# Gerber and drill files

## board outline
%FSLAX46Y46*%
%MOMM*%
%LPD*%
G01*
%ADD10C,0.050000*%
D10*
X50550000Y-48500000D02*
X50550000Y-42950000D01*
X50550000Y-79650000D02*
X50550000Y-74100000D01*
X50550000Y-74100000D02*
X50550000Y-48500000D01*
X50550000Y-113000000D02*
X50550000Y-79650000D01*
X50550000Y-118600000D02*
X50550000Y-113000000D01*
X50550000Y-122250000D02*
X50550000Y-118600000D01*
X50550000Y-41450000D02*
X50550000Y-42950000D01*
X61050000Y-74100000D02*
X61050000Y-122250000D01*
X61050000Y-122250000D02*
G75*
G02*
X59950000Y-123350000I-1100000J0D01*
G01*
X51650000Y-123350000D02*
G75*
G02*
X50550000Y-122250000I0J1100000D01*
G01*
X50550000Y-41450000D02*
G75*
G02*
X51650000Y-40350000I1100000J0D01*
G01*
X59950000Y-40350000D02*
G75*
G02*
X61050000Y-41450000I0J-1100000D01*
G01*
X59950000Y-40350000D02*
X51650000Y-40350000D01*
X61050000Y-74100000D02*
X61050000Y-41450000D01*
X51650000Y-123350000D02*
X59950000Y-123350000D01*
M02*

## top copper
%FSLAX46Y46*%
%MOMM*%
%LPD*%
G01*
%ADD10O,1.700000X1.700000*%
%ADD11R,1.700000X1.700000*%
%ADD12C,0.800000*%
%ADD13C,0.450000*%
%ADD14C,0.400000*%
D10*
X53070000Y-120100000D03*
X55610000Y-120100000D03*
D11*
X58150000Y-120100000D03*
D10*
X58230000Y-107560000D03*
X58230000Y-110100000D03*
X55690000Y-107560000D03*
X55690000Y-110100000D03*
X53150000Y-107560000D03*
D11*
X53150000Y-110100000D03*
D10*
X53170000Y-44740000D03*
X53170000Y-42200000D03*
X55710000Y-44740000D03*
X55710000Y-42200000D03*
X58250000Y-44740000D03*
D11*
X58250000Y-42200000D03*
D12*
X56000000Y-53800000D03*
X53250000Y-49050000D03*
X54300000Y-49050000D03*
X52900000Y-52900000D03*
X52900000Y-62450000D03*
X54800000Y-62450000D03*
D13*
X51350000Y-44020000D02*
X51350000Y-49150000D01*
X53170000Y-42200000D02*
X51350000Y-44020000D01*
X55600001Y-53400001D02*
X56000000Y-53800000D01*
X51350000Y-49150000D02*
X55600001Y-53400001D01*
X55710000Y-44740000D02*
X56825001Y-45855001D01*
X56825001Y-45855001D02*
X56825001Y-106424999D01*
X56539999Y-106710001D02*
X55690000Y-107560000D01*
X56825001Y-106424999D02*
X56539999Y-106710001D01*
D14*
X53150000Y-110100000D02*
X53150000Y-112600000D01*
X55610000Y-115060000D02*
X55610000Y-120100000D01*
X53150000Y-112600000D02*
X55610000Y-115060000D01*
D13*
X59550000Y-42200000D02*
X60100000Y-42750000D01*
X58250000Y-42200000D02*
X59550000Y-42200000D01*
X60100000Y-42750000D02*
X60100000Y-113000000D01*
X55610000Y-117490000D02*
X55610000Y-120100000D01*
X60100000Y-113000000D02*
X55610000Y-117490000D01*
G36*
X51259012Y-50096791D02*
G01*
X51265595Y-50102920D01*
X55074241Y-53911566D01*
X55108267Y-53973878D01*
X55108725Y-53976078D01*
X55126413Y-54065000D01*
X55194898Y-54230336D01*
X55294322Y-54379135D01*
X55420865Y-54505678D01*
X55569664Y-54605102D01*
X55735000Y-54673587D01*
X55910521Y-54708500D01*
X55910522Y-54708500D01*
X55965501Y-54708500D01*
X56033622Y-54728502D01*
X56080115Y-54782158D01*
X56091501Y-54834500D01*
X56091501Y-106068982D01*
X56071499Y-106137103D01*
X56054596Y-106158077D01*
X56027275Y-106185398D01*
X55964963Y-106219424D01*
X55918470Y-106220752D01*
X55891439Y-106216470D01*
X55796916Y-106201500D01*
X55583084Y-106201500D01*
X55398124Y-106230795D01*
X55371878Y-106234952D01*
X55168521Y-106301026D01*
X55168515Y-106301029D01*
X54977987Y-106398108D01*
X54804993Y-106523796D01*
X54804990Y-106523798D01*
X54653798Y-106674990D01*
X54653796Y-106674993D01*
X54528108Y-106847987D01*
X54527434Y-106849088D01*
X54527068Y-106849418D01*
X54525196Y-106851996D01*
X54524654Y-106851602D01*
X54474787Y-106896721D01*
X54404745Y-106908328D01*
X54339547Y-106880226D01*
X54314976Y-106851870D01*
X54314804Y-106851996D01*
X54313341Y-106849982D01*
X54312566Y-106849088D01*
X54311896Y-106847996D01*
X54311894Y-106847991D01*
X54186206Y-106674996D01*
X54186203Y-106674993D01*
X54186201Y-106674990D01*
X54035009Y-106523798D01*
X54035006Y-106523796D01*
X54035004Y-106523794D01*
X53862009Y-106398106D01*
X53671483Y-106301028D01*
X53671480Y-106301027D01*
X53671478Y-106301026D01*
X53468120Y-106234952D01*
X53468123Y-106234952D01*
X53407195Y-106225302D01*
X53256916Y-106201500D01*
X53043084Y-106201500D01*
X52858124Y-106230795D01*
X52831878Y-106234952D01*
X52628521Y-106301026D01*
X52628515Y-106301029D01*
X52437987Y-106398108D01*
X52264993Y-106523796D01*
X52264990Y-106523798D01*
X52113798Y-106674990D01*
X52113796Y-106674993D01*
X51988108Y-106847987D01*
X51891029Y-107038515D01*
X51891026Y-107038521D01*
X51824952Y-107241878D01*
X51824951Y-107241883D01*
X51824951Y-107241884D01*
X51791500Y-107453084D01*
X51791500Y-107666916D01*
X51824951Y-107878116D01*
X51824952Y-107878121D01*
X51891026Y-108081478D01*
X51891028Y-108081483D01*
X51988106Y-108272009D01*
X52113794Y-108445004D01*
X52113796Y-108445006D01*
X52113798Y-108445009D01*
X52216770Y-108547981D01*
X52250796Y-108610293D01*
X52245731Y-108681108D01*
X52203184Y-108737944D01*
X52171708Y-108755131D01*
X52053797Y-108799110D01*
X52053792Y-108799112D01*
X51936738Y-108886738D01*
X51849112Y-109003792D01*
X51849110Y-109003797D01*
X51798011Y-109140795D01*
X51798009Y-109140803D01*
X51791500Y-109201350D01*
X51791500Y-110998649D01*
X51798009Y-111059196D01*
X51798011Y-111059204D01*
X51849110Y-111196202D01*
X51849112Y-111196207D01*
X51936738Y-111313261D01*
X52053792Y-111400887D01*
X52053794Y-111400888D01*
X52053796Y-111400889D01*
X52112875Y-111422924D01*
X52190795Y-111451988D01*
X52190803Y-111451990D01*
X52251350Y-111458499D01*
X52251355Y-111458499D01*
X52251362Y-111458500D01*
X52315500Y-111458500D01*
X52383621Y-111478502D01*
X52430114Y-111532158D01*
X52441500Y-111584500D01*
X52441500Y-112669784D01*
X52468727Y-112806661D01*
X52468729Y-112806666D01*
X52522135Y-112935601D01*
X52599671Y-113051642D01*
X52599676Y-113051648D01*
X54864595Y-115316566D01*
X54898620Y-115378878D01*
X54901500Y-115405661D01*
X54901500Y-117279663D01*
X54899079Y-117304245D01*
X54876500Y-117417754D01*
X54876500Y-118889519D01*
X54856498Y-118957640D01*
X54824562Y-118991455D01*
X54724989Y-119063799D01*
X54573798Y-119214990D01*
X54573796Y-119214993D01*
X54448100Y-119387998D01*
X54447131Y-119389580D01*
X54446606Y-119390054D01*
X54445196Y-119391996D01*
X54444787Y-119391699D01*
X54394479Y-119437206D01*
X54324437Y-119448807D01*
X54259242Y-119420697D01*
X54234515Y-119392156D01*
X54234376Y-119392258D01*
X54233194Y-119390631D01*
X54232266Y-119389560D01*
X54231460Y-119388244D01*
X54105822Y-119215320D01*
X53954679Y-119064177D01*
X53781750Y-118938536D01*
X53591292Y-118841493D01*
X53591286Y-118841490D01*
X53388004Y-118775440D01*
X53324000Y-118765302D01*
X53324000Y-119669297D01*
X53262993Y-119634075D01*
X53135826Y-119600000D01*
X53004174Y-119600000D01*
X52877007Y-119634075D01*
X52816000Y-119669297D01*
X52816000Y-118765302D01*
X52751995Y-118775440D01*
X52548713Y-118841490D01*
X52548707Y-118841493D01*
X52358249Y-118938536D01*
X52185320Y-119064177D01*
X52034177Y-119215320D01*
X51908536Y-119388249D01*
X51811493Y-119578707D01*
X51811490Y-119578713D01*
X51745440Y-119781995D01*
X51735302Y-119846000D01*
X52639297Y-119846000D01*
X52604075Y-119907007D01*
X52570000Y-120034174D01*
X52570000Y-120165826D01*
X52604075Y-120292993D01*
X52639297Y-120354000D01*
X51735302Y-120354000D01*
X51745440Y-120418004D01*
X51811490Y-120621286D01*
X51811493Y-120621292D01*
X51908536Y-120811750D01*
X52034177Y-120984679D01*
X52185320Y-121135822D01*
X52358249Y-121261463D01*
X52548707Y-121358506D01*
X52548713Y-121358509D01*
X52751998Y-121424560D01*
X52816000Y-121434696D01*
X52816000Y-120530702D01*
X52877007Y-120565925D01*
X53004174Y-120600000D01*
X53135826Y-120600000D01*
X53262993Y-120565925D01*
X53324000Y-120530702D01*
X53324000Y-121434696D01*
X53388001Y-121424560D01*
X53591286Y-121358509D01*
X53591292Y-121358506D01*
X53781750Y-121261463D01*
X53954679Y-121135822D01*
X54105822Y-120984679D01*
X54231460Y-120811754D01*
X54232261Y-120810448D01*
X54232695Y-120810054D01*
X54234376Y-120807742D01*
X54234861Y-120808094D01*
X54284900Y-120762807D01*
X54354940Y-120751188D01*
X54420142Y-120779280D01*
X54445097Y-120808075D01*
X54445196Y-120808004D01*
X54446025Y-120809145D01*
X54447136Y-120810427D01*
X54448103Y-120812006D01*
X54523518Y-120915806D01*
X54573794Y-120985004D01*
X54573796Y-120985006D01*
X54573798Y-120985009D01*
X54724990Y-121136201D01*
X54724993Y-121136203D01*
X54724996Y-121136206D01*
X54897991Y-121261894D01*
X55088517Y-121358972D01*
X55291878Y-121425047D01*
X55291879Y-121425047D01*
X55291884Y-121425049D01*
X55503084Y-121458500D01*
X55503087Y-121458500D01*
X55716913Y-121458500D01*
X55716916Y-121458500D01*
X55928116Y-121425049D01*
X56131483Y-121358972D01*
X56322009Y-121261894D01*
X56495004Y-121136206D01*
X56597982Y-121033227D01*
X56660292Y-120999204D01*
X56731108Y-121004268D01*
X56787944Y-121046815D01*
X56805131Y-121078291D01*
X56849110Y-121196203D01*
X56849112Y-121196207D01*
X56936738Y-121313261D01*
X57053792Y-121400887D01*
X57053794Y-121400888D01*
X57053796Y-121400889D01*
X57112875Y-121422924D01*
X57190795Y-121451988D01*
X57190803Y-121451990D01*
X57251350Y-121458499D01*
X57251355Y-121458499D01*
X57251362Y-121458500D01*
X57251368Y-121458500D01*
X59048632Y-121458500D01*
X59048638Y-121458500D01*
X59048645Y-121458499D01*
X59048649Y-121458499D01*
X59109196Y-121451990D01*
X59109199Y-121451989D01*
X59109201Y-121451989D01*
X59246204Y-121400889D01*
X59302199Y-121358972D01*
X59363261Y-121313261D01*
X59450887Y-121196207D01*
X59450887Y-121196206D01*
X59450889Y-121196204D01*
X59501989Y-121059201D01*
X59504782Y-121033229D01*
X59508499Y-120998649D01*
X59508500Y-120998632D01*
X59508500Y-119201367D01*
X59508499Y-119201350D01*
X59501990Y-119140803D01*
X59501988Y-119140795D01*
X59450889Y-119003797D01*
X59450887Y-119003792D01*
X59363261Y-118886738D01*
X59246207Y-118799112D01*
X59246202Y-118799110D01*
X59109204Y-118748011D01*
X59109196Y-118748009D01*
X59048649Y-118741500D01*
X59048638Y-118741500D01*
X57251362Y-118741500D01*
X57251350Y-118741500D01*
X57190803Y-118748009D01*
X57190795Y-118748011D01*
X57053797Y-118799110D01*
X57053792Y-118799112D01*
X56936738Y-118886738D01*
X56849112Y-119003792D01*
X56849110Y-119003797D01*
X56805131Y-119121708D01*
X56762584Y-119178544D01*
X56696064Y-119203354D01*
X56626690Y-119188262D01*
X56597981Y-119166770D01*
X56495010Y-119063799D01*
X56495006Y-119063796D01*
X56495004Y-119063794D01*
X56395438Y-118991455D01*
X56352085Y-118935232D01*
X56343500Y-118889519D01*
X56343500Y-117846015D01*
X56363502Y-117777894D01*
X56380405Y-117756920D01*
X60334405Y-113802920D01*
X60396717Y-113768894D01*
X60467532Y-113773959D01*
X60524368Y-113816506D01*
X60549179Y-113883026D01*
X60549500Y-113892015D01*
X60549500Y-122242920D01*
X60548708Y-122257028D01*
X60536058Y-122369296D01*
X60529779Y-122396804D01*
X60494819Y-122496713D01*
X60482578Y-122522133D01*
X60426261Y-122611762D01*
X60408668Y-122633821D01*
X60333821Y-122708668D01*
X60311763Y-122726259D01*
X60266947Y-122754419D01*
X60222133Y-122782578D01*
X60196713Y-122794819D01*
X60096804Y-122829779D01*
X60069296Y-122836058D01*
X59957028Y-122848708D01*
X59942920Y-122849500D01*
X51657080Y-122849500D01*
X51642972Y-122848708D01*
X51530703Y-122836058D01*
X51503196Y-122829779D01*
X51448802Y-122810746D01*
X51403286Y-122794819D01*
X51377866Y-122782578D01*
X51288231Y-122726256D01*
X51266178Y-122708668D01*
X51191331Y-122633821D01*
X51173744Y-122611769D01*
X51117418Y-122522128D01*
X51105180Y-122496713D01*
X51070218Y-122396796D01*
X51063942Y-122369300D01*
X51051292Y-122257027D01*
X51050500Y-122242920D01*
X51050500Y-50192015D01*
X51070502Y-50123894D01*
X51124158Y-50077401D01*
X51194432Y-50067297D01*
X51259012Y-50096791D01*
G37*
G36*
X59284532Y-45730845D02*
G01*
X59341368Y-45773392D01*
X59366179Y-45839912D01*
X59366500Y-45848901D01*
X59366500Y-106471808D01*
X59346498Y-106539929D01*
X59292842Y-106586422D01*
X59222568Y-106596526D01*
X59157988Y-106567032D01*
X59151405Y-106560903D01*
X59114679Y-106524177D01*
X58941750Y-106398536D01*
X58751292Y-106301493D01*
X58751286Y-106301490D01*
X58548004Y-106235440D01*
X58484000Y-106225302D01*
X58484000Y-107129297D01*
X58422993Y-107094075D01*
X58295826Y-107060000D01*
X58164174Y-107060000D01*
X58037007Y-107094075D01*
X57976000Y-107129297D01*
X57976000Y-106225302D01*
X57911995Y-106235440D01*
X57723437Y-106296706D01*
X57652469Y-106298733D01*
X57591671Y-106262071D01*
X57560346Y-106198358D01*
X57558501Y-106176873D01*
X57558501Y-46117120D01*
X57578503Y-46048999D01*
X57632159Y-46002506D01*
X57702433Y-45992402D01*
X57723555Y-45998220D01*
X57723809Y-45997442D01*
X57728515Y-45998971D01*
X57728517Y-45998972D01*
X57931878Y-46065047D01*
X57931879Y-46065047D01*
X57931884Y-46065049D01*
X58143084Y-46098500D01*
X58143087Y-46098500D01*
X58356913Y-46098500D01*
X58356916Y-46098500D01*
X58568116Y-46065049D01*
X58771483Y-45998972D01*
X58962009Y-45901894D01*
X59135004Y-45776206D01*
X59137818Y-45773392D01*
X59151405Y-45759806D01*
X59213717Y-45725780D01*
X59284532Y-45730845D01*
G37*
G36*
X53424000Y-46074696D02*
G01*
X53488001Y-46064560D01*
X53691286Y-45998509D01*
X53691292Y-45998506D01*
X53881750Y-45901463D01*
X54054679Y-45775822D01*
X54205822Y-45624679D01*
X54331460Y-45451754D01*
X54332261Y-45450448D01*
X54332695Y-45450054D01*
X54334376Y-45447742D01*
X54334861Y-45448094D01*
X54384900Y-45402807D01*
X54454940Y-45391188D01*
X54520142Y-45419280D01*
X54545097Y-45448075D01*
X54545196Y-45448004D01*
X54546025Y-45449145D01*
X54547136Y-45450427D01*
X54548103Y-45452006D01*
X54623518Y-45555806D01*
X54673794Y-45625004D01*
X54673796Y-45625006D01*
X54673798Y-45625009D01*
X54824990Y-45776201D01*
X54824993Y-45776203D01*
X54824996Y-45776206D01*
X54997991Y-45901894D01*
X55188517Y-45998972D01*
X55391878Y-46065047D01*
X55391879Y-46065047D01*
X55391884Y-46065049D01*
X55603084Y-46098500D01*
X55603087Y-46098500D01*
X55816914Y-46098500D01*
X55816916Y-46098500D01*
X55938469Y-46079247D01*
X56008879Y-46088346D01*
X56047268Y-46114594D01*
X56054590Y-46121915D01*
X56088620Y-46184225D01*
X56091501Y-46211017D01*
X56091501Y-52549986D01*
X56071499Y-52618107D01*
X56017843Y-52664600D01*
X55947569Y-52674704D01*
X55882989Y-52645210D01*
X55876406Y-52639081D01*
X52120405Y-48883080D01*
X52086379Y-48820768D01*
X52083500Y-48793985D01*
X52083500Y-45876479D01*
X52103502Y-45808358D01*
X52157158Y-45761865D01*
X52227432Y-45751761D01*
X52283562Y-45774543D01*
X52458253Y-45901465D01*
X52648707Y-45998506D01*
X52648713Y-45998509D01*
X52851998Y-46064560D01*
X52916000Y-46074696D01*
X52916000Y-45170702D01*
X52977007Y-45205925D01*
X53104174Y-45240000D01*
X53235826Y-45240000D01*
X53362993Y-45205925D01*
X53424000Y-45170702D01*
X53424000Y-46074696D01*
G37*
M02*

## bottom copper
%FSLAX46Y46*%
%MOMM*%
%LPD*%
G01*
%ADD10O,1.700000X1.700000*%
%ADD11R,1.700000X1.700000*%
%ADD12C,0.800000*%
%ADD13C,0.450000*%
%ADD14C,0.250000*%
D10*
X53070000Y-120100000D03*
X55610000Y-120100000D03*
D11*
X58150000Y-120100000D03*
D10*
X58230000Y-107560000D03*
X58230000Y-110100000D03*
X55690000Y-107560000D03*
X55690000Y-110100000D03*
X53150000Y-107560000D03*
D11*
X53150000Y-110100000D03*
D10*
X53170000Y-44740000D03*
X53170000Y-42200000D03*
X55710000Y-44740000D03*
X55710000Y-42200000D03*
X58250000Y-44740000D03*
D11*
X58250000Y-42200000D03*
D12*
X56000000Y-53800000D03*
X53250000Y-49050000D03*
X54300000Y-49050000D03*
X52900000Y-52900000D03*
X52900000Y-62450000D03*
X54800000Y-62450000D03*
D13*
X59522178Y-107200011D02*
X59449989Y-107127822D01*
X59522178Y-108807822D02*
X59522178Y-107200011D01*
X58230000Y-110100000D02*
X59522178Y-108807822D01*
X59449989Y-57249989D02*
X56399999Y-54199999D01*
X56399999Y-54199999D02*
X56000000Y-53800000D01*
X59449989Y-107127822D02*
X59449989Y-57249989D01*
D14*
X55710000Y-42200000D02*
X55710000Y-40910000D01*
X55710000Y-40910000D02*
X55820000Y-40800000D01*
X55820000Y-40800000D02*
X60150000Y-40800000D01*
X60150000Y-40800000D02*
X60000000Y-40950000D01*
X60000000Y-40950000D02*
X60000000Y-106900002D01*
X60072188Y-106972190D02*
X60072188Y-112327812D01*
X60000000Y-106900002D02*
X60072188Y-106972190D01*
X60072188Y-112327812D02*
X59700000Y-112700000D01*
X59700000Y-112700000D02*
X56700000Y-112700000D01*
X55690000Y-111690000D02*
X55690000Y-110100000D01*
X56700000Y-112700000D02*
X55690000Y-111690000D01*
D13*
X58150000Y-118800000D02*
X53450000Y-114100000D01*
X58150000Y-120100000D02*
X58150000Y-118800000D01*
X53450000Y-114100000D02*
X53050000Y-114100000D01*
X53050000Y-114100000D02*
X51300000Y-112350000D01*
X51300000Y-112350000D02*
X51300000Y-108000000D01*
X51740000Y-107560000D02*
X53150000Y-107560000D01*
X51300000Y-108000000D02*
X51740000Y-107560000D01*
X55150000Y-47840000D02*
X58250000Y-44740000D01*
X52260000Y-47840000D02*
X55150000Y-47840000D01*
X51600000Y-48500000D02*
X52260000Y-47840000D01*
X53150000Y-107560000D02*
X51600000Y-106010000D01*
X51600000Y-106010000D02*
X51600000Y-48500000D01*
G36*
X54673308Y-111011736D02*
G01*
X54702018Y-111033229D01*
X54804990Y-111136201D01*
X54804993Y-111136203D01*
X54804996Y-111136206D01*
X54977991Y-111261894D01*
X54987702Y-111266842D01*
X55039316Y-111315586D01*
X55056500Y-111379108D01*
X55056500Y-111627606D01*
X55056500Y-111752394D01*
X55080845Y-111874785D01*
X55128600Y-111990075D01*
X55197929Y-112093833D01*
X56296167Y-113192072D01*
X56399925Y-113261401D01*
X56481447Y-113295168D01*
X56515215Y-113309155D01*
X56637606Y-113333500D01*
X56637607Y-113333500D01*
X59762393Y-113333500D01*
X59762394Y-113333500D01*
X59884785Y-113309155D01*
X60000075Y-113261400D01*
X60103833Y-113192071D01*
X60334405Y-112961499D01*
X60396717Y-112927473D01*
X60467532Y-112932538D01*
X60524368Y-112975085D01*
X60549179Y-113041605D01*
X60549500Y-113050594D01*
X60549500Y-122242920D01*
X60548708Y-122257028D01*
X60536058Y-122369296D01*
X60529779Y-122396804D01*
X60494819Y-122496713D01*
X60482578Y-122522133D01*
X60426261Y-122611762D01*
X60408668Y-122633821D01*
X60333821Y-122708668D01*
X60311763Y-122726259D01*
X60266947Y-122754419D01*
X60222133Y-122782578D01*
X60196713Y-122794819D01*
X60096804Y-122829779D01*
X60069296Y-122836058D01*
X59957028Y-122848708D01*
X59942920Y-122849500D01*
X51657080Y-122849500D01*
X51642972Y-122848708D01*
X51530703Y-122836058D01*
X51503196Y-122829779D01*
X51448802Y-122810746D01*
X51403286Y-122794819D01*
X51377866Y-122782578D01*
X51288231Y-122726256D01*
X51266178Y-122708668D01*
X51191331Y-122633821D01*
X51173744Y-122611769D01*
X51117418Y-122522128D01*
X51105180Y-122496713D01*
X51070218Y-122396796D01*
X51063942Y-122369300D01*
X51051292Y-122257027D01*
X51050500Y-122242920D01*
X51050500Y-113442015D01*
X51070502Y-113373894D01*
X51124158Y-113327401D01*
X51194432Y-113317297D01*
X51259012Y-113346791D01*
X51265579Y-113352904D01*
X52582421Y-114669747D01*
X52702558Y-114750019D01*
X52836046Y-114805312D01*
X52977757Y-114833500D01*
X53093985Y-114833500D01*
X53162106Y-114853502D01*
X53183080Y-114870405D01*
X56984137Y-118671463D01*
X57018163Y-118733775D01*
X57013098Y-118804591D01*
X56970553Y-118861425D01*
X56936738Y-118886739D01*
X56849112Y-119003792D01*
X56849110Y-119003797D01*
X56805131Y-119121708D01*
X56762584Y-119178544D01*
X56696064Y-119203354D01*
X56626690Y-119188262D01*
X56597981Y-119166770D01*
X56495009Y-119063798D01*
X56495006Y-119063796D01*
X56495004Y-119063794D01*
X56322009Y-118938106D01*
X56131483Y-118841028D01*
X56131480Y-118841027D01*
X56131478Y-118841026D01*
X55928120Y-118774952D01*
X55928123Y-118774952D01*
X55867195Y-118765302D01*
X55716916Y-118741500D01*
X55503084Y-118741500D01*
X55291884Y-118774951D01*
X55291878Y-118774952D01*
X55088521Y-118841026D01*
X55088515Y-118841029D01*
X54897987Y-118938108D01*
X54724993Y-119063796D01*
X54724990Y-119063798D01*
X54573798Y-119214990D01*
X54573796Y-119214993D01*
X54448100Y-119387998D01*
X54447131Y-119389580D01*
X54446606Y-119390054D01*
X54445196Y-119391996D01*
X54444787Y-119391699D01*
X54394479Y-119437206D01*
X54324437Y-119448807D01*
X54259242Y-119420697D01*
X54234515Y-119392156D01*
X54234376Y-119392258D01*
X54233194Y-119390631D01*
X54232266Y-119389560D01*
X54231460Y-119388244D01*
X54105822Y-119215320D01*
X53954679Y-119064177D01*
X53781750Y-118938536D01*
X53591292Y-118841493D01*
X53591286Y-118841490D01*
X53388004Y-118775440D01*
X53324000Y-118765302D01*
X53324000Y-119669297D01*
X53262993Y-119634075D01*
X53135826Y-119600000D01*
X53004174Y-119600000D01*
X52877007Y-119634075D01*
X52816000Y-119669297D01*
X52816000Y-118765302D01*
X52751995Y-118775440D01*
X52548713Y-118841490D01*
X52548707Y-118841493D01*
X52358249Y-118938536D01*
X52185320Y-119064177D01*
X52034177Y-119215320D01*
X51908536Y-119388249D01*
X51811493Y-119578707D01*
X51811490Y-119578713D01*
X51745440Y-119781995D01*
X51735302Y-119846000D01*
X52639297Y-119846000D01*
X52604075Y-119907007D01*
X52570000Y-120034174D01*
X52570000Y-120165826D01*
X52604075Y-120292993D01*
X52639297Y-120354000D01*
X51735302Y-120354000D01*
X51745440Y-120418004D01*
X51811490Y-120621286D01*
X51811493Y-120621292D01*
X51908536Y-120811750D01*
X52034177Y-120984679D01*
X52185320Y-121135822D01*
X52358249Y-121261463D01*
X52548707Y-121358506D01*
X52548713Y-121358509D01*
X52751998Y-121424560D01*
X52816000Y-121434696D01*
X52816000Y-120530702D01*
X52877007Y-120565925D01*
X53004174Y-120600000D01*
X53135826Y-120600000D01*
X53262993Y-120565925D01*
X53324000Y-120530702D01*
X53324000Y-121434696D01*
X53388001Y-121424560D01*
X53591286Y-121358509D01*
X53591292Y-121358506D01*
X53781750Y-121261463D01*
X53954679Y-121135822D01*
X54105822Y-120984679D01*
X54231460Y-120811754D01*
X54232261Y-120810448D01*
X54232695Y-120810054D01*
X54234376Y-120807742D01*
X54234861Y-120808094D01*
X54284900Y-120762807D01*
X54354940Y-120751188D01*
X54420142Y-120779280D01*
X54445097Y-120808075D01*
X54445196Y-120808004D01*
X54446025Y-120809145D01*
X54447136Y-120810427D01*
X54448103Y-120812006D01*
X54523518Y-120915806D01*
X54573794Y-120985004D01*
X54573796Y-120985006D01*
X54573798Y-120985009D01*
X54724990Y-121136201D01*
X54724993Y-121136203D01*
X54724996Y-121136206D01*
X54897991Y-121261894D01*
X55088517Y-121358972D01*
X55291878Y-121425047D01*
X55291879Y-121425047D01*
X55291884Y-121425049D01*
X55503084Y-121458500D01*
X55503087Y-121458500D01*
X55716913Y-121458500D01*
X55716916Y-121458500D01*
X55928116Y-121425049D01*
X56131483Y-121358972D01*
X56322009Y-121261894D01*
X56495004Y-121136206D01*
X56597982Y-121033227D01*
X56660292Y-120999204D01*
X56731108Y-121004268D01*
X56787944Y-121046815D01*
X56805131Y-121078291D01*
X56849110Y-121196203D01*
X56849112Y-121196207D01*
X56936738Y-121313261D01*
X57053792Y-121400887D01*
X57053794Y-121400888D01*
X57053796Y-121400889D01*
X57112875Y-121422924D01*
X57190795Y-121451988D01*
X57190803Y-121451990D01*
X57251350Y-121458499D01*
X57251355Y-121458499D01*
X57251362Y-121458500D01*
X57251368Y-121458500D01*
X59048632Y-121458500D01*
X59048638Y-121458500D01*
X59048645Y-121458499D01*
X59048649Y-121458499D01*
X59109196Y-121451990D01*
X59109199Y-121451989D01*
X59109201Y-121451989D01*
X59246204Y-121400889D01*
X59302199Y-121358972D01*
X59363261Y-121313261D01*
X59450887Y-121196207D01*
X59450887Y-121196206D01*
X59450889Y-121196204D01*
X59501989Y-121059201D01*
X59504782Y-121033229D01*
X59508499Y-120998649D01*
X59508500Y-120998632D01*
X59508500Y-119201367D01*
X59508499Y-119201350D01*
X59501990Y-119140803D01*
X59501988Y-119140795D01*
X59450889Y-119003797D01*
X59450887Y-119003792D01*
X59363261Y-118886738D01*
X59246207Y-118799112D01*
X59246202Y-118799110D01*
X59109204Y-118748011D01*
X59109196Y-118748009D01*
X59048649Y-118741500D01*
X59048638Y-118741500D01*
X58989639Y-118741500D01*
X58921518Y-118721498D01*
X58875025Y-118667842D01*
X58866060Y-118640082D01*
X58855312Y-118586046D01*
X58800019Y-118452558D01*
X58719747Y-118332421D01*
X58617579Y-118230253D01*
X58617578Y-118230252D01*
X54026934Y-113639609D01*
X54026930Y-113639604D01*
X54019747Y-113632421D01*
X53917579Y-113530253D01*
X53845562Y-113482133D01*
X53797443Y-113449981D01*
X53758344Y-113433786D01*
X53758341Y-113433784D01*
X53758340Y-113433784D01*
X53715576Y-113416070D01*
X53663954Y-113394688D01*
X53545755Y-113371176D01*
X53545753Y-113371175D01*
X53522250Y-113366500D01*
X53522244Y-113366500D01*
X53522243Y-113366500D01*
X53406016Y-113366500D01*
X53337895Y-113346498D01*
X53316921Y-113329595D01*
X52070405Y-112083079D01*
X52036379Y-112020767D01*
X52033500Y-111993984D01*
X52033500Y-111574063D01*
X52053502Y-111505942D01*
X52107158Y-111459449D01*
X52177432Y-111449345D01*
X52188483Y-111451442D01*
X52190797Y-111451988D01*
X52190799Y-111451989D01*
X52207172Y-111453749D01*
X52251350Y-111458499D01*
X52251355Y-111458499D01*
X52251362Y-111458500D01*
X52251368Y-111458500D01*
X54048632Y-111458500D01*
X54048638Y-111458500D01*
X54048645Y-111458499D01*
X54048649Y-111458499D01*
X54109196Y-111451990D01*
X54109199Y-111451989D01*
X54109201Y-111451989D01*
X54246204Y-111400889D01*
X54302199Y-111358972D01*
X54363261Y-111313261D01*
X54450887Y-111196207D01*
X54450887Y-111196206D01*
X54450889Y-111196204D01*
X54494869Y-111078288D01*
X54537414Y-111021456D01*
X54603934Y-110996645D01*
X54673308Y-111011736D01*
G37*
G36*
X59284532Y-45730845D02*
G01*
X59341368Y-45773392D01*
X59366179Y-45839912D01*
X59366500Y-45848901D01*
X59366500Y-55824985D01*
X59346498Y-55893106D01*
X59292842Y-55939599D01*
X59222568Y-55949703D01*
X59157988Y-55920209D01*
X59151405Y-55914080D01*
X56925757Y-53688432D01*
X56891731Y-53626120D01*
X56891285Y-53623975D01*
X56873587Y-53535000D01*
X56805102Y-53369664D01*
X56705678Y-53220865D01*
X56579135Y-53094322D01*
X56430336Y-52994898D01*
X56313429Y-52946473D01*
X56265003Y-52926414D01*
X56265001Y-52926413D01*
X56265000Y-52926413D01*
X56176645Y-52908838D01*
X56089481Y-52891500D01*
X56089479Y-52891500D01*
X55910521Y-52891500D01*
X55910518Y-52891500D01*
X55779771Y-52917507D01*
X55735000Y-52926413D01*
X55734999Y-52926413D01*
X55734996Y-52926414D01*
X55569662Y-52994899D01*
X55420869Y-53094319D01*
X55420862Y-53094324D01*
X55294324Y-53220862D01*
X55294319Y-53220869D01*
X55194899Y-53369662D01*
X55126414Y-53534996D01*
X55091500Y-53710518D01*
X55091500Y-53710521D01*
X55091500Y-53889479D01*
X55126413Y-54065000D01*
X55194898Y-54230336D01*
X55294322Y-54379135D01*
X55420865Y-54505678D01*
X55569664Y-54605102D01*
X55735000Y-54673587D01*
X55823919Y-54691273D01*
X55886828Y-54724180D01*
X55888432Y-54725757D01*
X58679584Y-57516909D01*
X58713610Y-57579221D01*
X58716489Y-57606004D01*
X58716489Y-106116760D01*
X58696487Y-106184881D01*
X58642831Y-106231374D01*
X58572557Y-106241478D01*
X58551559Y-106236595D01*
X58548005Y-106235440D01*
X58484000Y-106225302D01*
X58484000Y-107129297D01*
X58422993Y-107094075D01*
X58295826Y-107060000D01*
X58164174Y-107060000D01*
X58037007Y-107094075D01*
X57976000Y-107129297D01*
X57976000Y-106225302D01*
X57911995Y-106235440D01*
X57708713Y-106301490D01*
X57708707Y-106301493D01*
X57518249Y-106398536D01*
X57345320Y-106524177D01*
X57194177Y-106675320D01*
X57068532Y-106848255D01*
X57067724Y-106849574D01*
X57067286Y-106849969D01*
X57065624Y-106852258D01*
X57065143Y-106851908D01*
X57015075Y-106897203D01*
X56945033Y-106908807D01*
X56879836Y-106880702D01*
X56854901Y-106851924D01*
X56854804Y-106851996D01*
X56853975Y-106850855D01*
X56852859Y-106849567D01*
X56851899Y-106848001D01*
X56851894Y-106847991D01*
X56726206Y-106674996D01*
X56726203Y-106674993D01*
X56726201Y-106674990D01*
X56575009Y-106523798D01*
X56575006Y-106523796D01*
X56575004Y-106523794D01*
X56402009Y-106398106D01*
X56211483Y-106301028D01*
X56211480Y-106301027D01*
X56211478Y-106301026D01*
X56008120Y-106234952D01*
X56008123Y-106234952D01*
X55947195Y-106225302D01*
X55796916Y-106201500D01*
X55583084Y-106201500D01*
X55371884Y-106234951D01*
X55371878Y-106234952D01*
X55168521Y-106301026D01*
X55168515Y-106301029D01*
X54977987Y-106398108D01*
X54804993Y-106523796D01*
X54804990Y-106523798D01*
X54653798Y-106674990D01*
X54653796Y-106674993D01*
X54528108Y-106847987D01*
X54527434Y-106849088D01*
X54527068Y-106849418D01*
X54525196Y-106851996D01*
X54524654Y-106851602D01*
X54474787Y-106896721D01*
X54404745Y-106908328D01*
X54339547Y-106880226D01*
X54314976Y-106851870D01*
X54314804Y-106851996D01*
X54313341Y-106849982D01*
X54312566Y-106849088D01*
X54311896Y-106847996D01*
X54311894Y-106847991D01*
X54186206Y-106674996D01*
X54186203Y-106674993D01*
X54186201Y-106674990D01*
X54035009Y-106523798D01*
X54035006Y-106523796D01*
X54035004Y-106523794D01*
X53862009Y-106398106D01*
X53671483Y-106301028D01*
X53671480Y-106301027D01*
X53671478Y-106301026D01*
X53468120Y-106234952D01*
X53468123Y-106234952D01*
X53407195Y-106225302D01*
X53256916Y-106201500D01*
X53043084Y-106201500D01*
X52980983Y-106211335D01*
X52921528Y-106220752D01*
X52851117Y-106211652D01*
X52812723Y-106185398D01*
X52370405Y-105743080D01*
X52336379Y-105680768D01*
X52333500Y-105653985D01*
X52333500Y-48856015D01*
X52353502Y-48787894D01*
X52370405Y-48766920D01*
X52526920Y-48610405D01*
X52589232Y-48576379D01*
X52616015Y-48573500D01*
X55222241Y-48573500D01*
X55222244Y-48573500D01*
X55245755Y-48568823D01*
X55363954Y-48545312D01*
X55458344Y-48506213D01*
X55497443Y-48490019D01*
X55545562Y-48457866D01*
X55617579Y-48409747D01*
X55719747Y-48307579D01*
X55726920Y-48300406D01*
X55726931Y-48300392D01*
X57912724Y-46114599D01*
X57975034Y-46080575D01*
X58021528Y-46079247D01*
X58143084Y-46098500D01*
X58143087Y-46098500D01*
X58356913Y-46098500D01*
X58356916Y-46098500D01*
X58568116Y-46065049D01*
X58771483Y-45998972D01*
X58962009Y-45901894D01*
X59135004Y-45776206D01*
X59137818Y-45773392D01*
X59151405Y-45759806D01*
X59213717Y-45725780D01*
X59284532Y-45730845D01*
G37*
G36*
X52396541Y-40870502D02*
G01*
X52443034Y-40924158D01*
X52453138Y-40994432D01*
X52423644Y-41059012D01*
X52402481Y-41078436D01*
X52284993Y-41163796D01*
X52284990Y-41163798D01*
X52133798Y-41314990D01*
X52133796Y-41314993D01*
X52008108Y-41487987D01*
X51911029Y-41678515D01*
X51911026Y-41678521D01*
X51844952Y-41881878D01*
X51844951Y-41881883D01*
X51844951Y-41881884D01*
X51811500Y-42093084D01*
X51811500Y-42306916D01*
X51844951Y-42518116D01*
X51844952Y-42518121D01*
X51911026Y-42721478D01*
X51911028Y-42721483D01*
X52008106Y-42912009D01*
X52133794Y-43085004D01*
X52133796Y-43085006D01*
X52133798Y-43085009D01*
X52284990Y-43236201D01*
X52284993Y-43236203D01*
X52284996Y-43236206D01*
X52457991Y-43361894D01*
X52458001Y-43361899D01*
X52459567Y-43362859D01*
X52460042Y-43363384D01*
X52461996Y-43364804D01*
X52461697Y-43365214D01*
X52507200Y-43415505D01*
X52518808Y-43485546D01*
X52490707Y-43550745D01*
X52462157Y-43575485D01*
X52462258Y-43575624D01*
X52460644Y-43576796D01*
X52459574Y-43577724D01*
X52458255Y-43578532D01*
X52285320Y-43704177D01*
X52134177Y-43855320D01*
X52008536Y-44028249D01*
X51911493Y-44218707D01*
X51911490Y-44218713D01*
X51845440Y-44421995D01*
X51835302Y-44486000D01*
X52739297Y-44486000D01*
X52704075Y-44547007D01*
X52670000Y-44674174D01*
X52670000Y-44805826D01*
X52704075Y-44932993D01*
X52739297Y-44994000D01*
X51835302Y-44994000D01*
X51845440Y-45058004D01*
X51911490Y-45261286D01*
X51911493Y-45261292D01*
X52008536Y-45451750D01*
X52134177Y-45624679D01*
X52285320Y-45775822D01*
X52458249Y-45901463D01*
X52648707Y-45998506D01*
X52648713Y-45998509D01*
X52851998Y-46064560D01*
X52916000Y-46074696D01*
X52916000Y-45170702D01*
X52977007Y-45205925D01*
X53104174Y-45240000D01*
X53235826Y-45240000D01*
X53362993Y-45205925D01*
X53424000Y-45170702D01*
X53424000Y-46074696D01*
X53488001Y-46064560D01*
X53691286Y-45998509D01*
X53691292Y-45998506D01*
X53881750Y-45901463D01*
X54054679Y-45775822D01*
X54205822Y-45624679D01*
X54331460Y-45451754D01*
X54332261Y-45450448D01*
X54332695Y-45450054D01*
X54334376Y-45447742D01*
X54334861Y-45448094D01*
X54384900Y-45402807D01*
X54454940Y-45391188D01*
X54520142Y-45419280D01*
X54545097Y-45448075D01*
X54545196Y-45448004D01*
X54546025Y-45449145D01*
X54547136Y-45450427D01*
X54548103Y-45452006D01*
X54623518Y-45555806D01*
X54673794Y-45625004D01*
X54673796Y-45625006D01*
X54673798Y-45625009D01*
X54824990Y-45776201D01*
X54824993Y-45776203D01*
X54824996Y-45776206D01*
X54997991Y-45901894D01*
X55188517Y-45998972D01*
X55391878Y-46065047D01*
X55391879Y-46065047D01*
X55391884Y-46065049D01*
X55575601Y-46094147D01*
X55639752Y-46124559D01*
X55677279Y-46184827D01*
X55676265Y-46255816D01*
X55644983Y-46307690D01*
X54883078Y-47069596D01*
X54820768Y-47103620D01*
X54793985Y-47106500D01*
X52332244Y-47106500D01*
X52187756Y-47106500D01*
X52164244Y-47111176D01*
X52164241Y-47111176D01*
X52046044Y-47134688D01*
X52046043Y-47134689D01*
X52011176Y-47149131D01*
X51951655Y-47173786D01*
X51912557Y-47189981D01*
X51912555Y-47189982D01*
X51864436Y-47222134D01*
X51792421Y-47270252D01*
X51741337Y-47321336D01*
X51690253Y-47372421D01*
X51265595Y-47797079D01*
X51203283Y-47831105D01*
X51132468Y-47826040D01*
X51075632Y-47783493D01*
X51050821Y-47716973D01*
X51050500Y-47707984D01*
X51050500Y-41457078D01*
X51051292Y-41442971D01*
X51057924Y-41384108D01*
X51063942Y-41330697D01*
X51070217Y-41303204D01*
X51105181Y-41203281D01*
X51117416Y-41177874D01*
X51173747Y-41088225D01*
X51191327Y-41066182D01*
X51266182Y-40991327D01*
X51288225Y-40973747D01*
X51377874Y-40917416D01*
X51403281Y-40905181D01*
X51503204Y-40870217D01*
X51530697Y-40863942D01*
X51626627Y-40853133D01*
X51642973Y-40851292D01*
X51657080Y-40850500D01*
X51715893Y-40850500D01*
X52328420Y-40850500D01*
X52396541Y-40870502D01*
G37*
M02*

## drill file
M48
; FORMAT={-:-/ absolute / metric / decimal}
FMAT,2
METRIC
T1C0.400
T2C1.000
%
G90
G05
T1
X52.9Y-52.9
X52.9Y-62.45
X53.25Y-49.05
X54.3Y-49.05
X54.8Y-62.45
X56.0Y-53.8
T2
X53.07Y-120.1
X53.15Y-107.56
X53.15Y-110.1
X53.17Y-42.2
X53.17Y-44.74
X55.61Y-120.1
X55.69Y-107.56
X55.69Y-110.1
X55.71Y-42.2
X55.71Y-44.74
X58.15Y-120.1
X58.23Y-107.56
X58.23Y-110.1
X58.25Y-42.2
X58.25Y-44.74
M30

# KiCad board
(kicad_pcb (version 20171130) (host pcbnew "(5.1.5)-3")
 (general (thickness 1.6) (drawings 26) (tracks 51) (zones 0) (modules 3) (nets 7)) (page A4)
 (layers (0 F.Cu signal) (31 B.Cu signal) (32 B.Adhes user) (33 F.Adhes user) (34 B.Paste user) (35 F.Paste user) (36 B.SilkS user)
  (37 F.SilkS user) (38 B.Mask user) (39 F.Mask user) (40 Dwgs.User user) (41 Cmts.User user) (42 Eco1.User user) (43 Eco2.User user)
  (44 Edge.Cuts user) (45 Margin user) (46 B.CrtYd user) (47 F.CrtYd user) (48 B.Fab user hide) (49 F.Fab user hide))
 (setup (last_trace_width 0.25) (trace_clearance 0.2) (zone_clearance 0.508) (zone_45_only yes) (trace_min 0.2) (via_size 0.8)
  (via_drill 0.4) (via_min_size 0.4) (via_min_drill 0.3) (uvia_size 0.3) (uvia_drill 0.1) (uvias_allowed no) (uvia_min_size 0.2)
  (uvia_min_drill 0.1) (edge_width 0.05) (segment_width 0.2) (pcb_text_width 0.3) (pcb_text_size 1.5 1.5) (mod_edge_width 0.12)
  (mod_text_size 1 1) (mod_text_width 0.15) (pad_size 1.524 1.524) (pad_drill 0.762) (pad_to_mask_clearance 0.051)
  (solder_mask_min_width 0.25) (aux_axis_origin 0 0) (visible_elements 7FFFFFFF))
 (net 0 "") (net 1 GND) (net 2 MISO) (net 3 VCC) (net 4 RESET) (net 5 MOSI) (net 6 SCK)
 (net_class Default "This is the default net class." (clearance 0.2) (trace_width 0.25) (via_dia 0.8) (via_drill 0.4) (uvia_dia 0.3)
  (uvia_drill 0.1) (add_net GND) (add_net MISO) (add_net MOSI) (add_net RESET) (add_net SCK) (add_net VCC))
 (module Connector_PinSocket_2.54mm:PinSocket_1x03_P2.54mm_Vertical (layer B.Cu) (at 58.15 120.1 90)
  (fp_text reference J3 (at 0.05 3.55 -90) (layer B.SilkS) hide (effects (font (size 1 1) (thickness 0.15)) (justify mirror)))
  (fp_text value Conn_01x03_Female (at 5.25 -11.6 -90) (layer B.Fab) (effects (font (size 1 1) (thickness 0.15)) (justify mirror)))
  (pad 3 thru_hole oval (at 0 -5.08 90) (size 1.7 1.7) (drill 1) (layers *.Cu *.Mask) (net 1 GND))
  (pad 2 thru_hole oval (at 0 -2.54 90) (size 1.7 1.7) (drill 1) (layers *.Cu *.Mask) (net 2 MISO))
  (pad 1 thru_hole rect (at 0 0 90) (size 1.7 1.7) (drill 1) (layers *.Cu *.Mask) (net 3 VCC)))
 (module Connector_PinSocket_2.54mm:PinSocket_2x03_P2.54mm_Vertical (layer B.Cu) (at 53.15 110.1 270)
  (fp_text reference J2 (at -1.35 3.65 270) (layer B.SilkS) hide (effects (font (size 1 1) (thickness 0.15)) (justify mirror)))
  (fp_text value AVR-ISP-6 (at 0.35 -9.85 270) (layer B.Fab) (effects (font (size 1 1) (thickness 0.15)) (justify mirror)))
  (pad 6 thru_hole oval (at -2.54 -5.08 270) (size 1.7 1.7) (drill 1) (layers *.Cu *.Mask) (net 1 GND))
  (pad 5 thru_hole oval (at 0 -5.08 270) (size 1.7 1.7) (drill 1) (layers *.Cu *.Mask) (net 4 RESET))
  (pad 4 thru_hole oval (at -2.54 -2.54 270) (size 1.7 1.7) (drill 1) (layers *.Cu *.Mask) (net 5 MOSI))
  (pad 3 thru_hole oval (at 0 -2.54 270) (size 1.7 1.7) (drill 1) (layers *.Cu *.Mask) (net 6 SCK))
  (pad 2 thru_hole oval (at -2.54 0 270) (size 1.7 1.7) (drill 1) (layers *.Cu *.Mask) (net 3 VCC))
  (pad 1 thru_hole rect (at 0 0 270) (size 1.7 1.7) (drill 1) (layers *.Cu *.Mask) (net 2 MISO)))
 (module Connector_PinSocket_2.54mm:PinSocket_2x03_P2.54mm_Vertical (layer B.Cu) (at 58.25 42.2 90)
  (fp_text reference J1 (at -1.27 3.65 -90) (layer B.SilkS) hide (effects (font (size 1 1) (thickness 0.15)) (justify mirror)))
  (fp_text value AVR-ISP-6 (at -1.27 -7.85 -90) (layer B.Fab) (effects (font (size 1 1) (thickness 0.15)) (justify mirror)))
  (pad 6 thru_hole oval (at -2.54 -5.08 90) (size 1.7 1.7) (drill 1) (layers *.Cu *.Mask) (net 1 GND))
  (pad 5 thru_hole oval (at 0 -5.08 90) (size 1.7 1.7) (drill 1) (layers *.Cu *.Mask) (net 4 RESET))
  (pad 4 thru_hole oval (at -2.54 -2.54 90) (size 1.7 1.7) (drill 1) (layers *.Cu *.Mask) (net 5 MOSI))
  (pad 3 thru_hole oval (at 0 -2.54 90) (size 1.7 1.7) (drill 1) (layers *.Cu *.Mask) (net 6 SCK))
  (pad 2 thru_hole oval (at -2.54 0 90) (size 1.7 1.7) (drill 1) (layers *.Cu *.Mask) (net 3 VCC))
  (pad 1 thru_hole rect (at 0 0 90) (size 1.7 1.7) (drill 1) (layers *.Cu *.Mask) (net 2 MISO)))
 (gr_line (start 50.55 48.5) (end 50.55 42.95) (layer Edge.Cuts) (width 0.05))
 (gr_line (start 50.55 79.65) (end 50.55 74.1) (layer Edge.Cuts) (width 0.05))
 (gr_line (start 50.55 74.1) (end 50.55 48.5) (layer Edge.Cuts) (width 0.05))
 (gr_line (start 50.55 113) (end 50.55 79.65) (layer Edge.Cuts) (width 0.05))
 (gr_line (start 50.55 118.6) (end 50.55 113) (layer Edge.Cuts) (width 0.05))
 (gr_line (start 50.55 122.25) (end 50.55 118.6) (layer Edge.Cuts) (width 0.05))
 (gr_line (start 50.55 41.45) (end 50.55 42.95) (layer Edge.Cuts) (width 0.05))
 (gr_line (start 61.05 74.1) (end 61.05 122.25) (layer Edge.Cuts) (width 0.05))
 (gr_arc (start 59.95 122.25) (end 59.95 123.35) (angle -90) (layer Edge.Cuts) (width 0.05))
 (gr_arc (start 51.65 122.25) (end 50.55 122.25) (angle -90) (layer Edge.Cuts) (width 0.05))
 (gr_arc (start 51.65 41.45) (end 51.65 40.35) (angle -90) (layer Edge.Cuts) (width 0.05))
 (gr_arc (start 59.95 41.45) (end 61.05 41.45) (angle -90) (layer Edge.Cuts) (width 0.05))
 (gr_line (start 59.95 40.35) (end 51.65 40.35) (layer Edge.Cuts) (width 0.05))
 (gr_line (start 61.05 74.1) (end 61.05 41.45) (layer Edge.Cuts) (width 0.05))
 (gr_line (start 51.65 123.35) (end 59.95 123.35) (layer Edge.Cuts) (width 0.05))
 (segment (start 51.35 44.02) (end 51.35 49.15) (width 0.45) (layer F.Cu) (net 4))
 (segment (start 53.17 42.2) (end 51.35 44.02) (width 0.45) (layer F.Cu) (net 4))
 (segment (start 55.600001 53.400001) (end 56 53.8) (width 0.45) (layer F.Cu) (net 4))
 (via (at 56 53.8) (size 0.8) (drill 0.4) (layers F.Cu B.Cu) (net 4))
 (segment (start 51.35 49.15) (end 55.600001 53.400001) (width 0.45) (layer F.Cu) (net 4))
 (segment (start 59.522178 107.200011) (end 59.449989 107.127822) (width 0.45) (layer B.Cu) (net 4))
 (segment (start 59.522178 108.807822) (end 59.522178 107.200011) (width 0.45) (layer B.Cu) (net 4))
 (segment (start 58.23 110.1) (end 59.522178 108.807822) (width 0.45) (layer B.Cu) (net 4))
 (segment (start 59.449989 57.249989) (end 56.399999 54.199999) (width 0.45) (layer B.Cu) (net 4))
 (segment (start 56.399999 54.199999) (end 56 53.8) (width 0.45) (layer B.Cu) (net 4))
 (segment (start 59.449989 107.127822) (end 59.449989 57.249989) (width 0.45) (layer B.Cu) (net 4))
 (segment (start 55.71 44.74) (end 56.825001 45.855001) (width 0.45) (layer F.Cu) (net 5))
 (segment (start 56.825001 45.855001) (end 56.825001 106.424999) (width 0.45) (layer F.Cu) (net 5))
 (segment (start 56.539999 106.710001) (end 55.69 107.56) (width 0.45) (layer F.Cu) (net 5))
 (segment (start 56.825001 106.424999) (end 56.539999 106.710001) (width 0.45) (layer F.Cu) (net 5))
 (segment (start 55.71 42.2) (end 55.71 40.91) (width 0.25) (layer B.Cu) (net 6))
 (segment (start 55.71 40.91) (end 55.82 40.8) (width 0.25) (layer B.Cu) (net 6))
 (segment (start 55.82 40.8) (end 60.15 40.8) (width 0.25) (layer B.Cu) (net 6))
 (segment (start 60.15 40.8) (end 60 40.95) (width 0.25) (layer B.Cu) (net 6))
 (segment (start 60 40.95) (end 60 106.900002) (width 0.25) (layer B.Cu) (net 6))
 (segment (start 60.072188 106.97219) (end 60.072188 112.327812) (width 0.25) (layer B.Cu) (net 6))
 (segment (start 60 106.900002) (end 60.072188 106.97219) (width 0.25) (layer B.Cu) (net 6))
 (segment (start 60.072188 112.327812) (end 59.7 112.7) (width 0.25) (layer B.Cu) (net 6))
 (segment (start 59.7 112.7) (end 56.7 112.7) (width 0.25) (layer B.Cu) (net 6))
 (segment (start 55.69 111.69) (end 55.69 110.1) (width 0.25) (layer B.Cu) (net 6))
 (segment (start 56.7 112.7) (end 55.69 111.69) (width 0.25) (layer B.Cu) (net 6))
 (segment (start 58.15 118.8) (end 53.45 114.1) (width 0.45) (layer B.Cu) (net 3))
 (segment (start 58.15 120.1) (end 58.15 118.8) (width 0.45) (layer B.Cu) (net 3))
 (segment (start 53.45 114.1) (end 53.05 114.1) (width 0.45) (layer B.Cu) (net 3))
 (segment (start 53.05 114.1) (end 51.3 112.35) (width 0.45) (layer B.Cu) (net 3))
 (segment (start 51.3 112.35) (end 51.3 108) (width 0.45) (layer B.Cu) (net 3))
 (segment (start 51.74 107.56) (end 53.15 107.56) (width 0.45) (layer B.Cu) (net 3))
 (segment (start 51.3 108) (end 51.74 107.56) (width 0.45) (layer B.Cu) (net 3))
 (segment (start 55.15 47.84) (end 58.25 44.74) (width 0.45) (layer B.Cu) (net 3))
 (segment (start 52.26 47.84) (end 55.15 47.84) (width 0.45) (layer B.Cu) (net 3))
 (segment (start 51.6 48.5) (end 52.26 47.84) (width 0.45) (layer B.Cu) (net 3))
 (segment (start 53.15 107.56) (end 51.6 106.01) (width 0.45) (layer B.Cu) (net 3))
 (segment (start 51.6 106.01) (end 51.6 48.5) (width 0.45) (layer B.Cu) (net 3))
 (segment (start 53.15 110.1) (end 53.15 112.6) (width 0.4) (layer F.Cu) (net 2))
 (segment (start 55.61 115.06) (end 55.61 120.1) (width 0.4) (layer F.Cu) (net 2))
 (segment (start 53.15 112.6) (end 55.61 115.06) (width 0.4) (layer F.Cu) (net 2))
 (segment (start 59.55 42.2) (end 60.1 42.75) (width 0.45) (layer F.Cu) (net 2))
 (segment (start 58.25 42.2) (end 59.55 42.2) (width 0.45) (layer F.Cu) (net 2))
 (segment (start 60.1 42.75) (end 60.1 113) (width 0.45) (layer F.Cu) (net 2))
 (segment (start 55.61 117.49) (end 55.61 120.1) (width 0.45) (layer F.Cu) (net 2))
 (segment (start 60.1 113) (end 55.61 117.49) (width 0.45) (layer F.Cu) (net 2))
 (via (at 53.25 49.05) (size 0.8) (drill 0.4) (layers F.Cu B.Cu) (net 1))
 (via (at 54.3 49.05) (size 0.8) (drill 0.4) (layers F.Cu B.Cu) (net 1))
 (via (at 52.9 52.9) (size 0.8) (drill 0.4) (layers F.Cu B.Cu) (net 1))
 (via (at 52.9 62.45) (size 0.8) (drill 0.4) (layers F.Cu B.Cu) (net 1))
 (via (at 54.8 62.45) (size 0.8) (drill 0.4) (layers F.Cu B.Cu) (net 1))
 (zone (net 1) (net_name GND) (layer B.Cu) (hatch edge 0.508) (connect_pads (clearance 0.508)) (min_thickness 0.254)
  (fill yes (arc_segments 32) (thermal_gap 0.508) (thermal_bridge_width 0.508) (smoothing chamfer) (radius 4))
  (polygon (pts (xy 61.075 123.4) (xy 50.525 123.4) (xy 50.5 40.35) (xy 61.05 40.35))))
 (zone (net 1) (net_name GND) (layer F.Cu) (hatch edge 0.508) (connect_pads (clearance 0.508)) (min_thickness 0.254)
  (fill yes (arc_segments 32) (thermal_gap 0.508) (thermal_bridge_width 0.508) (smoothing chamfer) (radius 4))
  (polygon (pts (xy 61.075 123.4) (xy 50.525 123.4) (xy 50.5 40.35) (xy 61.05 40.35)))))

